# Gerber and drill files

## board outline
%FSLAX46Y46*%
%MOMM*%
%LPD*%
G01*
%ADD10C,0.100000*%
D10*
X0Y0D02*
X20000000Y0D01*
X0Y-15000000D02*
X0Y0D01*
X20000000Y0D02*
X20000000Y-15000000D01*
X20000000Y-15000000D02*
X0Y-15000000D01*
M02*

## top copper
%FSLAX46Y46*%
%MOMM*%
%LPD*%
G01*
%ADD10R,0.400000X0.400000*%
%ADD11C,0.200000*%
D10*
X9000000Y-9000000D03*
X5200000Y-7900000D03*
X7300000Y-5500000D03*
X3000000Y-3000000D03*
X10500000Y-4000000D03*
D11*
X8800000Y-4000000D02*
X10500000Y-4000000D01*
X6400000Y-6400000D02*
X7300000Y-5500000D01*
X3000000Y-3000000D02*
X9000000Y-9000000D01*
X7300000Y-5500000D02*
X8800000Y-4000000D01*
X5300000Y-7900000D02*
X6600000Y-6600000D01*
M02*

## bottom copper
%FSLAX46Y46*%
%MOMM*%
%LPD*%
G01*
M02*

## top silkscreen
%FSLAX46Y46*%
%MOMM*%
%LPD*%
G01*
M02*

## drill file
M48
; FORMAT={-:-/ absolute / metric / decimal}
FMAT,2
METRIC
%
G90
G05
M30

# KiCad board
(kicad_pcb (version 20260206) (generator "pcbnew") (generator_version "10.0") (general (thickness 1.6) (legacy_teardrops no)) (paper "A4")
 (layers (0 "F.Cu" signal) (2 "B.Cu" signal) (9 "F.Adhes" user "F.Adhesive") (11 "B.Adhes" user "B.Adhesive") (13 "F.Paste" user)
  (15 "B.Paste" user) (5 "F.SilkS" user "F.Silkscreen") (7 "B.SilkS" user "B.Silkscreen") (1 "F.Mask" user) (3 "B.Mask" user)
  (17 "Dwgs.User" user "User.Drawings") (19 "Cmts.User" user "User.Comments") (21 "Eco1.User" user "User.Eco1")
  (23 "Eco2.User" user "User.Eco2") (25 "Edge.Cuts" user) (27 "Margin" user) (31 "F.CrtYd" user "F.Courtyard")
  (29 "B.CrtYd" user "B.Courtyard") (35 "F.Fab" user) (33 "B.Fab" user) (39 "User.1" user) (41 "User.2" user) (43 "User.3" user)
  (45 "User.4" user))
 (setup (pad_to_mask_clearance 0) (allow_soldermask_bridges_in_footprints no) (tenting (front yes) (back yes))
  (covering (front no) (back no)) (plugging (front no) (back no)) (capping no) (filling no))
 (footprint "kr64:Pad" (layer "F.Cu") (at 9 9)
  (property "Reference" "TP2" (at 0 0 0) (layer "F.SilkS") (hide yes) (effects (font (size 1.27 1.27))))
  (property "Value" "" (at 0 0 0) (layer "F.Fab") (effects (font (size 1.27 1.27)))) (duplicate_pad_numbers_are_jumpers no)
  (pad "1" smd rect (at 0 0) (size 0.4 0.4) (layers "F.Cu" "F.Mask" "F.Paste") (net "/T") (thermal_bridge_angle 45)))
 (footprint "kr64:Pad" (layer "F.Cu") (at 5.2 7.9)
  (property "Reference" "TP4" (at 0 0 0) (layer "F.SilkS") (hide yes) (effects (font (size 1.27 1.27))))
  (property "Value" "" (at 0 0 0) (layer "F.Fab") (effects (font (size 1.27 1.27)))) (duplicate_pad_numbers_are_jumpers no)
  (pad "1" smd rect (at 0 0) (size 0.4 0.4) (layers "F.Cu" "F.Mask" "F.Paste") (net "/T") (thermal_bridge_angle 45)))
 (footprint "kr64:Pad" (layer "F.Cu") (at 7.3 5.5)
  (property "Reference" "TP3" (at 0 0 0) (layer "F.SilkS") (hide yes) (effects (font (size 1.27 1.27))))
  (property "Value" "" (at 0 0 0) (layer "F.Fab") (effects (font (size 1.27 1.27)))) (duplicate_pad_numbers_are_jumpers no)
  (pad "1" smd rect (at 0 0) (size 0.4 0.4) (layers "F.Cu" "F.Mask" "F.Paste") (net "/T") (thermal_bridge_angle 45)))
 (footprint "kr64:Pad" (layer "F.Cu") (at 3 3)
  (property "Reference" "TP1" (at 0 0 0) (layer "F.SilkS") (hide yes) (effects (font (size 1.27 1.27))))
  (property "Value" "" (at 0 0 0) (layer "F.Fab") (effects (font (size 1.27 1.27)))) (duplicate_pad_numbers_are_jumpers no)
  (pad "1" smd rect (at 0 0) (size 0.4 0.4) (layers "F.Cu" "F.Mask" "F.Paste") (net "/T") (thermal_bridge_angle 45)))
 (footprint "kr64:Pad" (layer "F.Cu") (at 10.5 4)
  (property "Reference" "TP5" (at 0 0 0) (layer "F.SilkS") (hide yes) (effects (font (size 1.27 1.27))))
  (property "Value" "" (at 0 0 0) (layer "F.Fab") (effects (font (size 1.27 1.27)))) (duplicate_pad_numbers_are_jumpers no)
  (pad "1" smd rect (at 0 0) (size 0.4 0.4) (layers "F.Cu" "F.Mask" "F.Paste") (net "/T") (thermal_bridge_angle 45)))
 (gr_line (start 0 0) (end 20 0) (stroke (width 0.1) (type default)) (layer "Edge.Cuts"))
 (gr_line (start 0 15) (end 0 0) (stroke (width 0.1) (type default)) (layer "Edge.Cuts"))
 (gr_line (start 20 0) (end 20 15) (stroke (width 0.1) (type default)) (layer "Edge.Cuts"))
 (gr_line (start 20 15) (end 0 15) (stroke (width 0.1) (type default)) (layer "Edge.Cuts"))
 (segment (start 8.8 4) (end 10.5 4) (width 0.2) (layer "F.Cu") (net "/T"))
 (segment (start 6.4 6.4) (end 7.3 5.5) (width 0.2) (layer "F.Cu") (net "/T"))
 (segment (start 3 3) (end 9 9) (width 0.2) (layer "F.Cu") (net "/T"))
 (segment (start 7.3 5.5) (end 8.8 4) (width 0.2) (layer "F.Cu") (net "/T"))
 (segment (start 5.3 7.9) (end 6.6 6.6) (width 0.2) (layer "F.Cu") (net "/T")))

